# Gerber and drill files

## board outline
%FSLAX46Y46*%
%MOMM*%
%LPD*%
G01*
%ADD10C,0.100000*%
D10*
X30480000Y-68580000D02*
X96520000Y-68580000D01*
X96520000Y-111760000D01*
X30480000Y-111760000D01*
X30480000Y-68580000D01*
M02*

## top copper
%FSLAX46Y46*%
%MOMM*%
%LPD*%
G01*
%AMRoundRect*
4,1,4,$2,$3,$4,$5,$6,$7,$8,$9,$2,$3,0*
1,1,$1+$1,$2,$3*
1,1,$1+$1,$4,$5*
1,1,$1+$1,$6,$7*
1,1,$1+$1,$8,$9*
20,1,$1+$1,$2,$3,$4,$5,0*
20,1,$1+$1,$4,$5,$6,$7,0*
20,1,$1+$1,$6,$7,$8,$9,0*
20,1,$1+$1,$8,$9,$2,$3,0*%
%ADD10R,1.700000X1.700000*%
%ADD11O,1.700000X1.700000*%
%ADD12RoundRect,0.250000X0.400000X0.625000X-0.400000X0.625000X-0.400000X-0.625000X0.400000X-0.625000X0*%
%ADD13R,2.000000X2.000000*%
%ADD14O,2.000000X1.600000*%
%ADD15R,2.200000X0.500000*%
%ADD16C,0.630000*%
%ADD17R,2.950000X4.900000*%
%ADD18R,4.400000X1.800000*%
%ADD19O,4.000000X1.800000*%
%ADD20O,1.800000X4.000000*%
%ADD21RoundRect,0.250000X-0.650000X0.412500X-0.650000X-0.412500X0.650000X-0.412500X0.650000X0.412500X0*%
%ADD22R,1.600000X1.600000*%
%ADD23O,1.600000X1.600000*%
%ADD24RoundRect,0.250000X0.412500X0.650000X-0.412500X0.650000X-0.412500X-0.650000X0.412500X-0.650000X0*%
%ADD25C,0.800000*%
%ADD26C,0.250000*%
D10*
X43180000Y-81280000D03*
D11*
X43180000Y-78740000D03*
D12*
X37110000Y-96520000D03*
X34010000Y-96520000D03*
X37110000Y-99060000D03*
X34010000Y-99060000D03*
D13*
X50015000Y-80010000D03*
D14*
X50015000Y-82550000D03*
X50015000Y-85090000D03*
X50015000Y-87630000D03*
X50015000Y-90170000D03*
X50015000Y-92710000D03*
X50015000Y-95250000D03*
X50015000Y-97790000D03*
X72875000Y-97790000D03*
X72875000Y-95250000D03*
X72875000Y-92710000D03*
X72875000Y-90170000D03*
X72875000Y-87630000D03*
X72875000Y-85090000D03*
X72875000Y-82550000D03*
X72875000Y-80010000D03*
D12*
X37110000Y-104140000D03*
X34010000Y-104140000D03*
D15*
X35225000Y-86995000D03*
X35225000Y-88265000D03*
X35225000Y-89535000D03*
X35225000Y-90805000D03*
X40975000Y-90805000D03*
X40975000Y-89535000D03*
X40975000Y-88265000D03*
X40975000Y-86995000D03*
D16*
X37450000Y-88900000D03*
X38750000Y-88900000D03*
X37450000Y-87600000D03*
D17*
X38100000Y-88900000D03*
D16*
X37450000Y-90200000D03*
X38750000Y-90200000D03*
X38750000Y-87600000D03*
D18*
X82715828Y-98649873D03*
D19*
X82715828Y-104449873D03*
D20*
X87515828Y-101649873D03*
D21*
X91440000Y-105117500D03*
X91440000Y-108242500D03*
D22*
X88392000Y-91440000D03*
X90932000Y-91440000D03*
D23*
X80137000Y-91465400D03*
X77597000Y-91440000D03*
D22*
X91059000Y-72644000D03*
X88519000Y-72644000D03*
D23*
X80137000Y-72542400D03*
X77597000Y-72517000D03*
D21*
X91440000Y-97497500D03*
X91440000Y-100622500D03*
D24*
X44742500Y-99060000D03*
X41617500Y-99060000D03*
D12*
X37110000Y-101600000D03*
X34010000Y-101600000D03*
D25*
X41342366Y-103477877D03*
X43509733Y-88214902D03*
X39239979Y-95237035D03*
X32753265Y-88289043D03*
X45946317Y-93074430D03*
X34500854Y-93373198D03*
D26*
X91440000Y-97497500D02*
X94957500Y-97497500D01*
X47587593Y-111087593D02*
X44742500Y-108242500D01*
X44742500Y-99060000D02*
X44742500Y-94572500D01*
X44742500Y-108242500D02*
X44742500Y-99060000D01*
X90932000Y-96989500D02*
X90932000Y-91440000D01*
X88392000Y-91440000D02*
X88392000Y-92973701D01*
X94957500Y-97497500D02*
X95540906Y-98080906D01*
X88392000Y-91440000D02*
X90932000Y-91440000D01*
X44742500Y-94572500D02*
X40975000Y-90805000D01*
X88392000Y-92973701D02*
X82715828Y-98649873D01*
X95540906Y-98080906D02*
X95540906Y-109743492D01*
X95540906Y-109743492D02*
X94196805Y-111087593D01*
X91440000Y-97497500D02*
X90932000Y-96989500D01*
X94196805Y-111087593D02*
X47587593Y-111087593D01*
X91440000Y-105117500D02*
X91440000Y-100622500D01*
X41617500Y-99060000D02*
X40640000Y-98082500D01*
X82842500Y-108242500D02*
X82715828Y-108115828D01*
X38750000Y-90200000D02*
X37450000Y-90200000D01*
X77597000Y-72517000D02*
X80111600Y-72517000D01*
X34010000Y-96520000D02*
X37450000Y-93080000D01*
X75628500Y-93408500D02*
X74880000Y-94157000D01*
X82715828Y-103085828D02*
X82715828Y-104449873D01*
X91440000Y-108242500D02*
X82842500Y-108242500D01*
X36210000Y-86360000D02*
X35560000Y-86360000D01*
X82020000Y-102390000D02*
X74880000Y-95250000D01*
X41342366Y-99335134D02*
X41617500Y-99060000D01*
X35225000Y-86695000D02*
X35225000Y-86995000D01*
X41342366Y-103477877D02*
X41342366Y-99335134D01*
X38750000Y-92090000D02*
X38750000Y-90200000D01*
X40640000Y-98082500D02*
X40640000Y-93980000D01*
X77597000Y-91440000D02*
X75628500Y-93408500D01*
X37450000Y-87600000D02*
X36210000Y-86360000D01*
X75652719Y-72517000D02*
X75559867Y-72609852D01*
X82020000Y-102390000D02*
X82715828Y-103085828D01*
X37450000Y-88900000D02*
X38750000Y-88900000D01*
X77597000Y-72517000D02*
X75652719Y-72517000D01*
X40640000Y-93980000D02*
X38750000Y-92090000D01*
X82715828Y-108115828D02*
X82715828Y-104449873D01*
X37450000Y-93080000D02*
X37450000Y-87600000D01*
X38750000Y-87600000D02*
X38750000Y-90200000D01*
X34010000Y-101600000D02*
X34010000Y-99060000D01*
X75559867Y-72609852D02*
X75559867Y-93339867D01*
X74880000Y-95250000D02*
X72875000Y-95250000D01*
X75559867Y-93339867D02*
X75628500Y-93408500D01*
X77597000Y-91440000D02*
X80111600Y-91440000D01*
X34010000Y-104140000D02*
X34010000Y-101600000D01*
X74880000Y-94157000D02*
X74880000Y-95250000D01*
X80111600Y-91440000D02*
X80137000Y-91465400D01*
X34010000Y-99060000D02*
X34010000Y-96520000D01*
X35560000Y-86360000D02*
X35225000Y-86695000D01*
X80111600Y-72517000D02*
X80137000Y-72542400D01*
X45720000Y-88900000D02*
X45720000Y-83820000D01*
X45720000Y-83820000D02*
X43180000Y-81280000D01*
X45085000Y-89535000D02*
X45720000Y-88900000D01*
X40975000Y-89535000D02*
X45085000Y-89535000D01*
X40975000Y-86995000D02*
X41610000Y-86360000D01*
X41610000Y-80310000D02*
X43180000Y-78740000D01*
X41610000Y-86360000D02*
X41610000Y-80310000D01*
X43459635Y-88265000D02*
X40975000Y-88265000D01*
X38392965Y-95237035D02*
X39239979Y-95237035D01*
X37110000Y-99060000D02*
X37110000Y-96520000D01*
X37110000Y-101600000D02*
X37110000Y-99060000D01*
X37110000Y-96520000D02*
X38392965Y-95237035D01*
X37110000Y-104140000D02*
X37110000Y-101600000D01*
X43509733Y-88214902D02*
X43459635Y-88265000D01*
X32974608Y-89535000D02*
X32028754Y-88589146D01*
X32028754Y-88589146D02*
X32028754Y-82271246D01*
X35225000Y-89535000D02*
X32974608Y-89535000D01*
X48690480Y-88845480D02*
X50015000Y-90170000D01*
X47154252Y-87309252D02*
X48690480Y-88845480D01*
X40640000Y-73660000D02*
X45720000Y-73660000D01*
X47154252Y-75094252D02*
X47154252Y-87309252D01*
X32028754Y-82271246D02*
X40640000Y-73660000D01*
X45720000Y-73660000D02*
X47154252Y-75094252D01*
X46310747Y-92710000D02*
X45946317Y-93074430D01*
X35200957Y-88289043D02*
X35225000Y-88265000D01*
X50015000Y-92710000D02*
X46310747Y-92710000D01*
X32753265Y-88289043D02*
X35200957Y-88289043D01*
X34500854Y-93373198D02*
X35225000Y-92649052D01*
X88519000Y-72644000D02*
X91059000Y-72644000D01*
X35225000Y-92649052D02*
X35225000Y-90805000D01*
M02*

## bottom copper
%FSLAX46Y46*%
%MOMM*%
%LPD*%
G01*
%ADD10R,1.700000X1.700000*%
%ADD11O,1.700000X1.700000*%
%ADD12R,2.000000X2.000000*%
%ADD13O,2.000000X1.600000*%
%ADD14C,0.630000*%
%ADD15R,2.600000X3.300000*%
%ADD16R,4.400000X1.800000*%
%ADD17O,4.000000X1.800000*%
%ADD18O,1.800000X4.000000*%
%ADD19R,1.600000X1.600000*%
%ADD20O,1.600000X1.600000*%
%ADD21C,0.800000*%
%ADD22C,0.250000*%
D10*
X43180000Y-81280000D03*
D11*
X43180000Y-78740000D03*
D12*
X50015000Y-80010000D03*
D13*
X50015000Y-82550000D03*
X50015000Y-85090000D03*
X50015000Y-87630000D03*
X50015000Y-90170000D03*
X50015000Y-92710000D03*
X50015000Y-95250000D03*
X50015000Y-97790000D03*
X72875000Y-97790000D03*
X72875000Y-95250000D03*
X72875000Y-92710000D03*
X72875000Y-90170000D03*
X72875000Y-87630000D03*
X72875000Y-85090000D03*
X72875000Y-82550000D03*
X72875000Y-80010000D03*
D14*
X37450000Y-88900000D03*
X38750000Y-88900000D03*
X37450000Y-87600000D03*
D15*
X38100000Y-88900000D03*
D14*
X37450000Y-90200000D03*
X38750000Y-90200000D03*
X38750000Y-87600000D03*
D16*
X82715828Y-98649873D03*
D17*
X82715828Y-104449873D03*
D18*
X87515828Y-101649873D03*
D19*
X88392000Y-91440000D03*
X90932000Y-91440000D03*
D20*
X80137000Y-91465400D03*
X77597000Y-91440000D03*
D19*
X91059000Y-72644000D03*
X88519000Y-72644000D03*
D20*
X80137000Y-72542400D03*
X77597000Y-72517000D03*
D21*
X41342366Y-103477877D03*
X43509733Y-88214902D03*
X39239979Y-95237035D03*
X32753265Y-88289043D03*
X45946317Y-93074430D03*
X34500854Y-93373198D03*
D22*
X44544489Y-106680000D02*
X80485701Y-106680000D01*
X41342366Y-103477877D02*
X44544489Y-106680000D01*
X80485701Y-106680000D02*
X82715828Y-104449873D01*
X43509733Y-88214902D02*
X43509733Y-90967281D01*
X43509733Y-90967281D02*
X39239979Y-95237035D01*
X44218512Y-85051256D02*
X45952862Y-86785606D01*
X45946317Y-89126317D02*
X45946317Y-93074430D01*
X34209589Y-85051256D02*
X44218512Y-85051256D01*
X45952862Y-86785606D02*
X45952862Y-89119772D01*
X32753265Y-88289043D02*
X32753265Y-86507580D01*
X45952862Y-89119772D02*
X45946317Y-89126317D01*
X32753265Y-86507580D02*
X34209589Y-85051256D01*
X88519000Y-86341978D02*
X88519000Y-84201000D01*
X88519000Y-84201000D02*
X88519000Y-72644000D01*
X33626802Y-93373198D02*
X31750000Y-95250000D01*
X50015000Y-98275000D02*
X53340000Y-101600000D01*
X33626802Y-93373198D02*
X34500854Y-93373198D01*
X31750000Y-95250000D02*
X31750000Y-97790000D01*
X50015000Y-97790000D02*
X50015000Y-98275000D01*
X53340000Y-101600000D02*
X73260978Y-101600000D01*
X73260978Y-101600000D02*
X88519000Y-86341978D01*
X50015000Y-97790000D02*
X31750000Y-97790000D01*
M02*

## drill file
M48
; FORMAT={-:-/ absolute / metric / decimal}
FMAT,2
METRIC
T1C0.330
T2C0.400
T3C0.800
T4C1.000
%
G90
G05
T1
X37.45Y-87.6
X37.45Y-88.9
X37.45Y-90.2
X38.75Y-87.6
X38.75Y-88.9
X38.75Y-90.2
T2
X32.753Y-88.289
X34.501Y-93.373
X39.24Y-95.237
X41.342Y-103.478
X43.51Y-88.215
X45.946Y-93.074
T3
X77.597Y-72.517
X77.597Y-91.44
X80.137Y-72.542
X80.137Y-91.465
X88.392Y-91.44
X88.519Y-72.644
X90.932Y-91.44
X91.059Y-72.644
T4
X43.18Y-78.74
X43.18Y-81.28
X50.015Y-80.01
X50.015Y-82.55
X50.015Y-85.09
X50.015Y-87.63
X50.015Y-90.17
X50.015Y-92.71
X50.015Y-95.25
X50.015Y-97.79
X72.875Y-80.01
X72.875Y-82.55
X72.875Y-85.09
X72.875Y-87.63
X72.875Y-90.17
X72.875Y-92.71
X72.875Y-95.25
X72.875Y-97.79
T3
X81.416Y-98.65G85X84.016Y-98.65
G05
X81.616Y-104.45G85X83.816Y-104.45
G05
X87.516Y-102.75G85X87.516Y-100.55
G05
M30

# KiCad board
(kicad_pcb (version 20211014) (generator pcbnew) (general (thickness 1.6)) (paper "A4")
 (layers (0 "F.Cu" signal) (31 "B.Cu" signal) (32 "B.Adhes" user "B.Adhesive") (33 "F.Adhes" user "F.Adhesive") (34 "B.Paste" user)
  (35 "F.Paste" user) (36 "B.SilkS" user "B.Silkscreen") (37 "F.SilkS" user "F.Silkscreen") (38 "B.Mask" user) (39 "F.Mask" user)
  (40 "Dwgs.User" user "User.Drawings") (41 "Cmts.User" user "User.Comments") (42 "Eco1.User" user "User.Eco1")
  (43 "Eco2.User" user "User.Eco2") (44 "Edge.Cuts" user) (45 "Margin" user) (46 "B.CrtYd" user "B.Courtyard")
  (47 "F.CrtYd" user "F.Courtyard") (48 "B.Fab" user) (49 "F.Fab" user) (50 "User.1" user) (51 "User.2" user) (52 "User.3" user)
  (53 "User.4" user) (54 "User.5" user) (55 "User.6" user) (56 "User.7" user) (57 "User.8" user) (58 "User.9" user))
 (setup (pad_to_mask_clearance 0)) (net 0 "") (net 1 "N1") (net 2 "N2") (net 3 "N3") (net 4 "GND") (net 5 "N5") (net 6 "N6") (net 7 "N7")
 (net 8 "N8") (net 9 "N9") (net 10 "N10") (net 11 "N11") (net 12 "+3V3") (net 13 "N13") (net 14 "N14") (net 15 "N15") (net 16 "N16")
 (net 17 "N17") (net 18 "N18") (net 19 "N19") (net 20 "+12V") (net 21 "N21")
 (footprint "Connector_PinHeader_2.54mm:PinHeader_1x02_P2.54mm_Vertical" (layer "F.Cu") (at 43.18 81.28 180)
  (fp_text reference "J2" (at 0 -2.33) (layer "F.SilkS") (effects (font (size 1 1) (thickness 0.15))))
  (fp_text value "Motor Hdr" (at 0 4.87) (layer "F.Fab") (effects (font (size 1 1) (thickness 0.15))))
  (pad "1" thru_hole rect (at 0 0 180) (size 1.7 1.7) (drill 1) (layers *.Cu *.Mask) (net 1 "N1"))
  (pad "2" thru_hole oval (at 0 2.54 180) (size 1.7 1.7) (drill 1) (layers *.Cu *.Mask) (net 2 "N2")))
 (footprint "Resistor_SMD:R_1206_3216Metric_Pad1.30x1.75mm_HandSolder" (layer "F.Cu") (at 35.56 96.52 180)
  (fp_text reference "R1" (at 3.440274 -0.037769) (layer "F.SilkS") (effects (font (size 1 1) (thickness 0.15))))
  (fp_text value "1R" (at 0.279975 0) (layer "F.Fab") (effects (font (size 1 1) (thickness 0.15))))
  (pad "1" smd roundrect (at -1.55 0 180) (size 1.3 1.75) (layers "F.Cu" "F.Paste" "F.Mask") (roundrect_rratio 0.1923076923) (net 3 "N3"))
  (pad "2" smd roundrect (at 1.55 0 180) (size 1.3 1.75) (layers "F.Cu" "F.Paste" "F.Mask") (roundrect_rratio 0.1923076923) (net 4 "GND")))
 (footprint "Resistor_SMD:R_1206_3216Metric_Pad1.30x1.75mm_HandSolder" (layer "F.Cu") (at 35.56 99.06 180)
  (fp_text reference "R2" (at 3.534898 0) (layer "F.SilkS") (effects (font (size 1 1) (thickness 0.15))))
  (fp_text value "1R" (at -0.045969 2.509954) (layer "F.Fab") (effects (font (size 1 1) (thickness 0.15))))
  (pad "1" smd roundrect (at -1.55 0 180) (size 1.3 1.75) (layers "F.Cu" "F.Paste" "F.Mask") (roundrect_rratio 0.1923076923) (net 3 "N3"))
  (pad "2" smd roundrect (at 1.55 0 180) (size 1.3 1.75) (layers "F.Cu" "F.Paste" "F.Mask") (roundrect_rratio 0.1923076923) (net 4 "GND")))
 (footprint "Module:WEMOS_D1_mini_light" (layer "F.Cu") (at 50.015 80.01)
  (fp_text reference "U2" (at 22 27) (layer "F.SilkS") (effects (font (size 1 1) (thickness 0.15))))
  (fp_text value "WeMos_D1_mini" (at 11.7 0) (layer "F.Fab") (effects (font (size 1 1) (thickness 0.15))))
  (pad "1" thru_hole rect (at 0 0) (size 2 2) (drill 1) (layers *.Cu *.Mask) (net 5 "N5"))
  (pad "2" thru_hole oval (at 0 2.54) (size 2 1.6) (drill 1) (layers *.Cu *.Mask) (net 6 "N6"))
  (pad "3" thru_hole oval (at 0 5.08) (size 2 1.6) (drill 1) (layers *.Cu *.Mask) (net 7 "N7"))
  (pad "4" thru_hole oval (at 0 7.62) (size 2 1.6) (drill 1) (layers *.Cu *.Mask) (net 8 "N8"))
  (pad "5" thru_hole oval (at 0 10.16) (size 2 1.6) (drill 1) (layers *.Cu *.Mask) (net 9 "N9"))
  (pad "6" thru_hole oval (at 0 12.7) (size 2 1.6) (drill 1) (layers *.Cu *.Mask) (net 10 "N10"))
  (pad "7" thru_hole oval (at 0 15.24) (size 2 1.6) (drill 1) (layers *.Cu *.Mask) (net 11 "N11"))
  (pad "8" thru_hole oval (at 0 17.78) (size 2 1.6) (drill 1) (layers *.Cu *.Mask) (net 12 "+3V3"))
  (pad "9" thru_hole oval (at 22.86 17.78) (size 2 1.6) (drill 1) (layers *.Cu *.Mask) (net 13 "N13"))
  (pad "10" thru_hole oval (at 22.86 15.24) (size 2 1.6) (drill 1) (layers *.Cu *.Mask) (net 4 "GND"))
  (pad "11" thru_hole oval (at 22.86 12.7) (size 2 1.6) (drill 1) (layers *.Cu *.Mask) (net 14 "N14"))
  (pad "12" thru_hole oval (at 22.86 10.16) (size 2 1.6) (drill 1) (layers *.Cu *.Mask) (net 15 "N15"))
  (pad "13" thru_hole oval (at 22.86 7.62) (size 2 1.6) (drill 1) (layers *.Cu *.Mask) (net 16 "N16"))
  (pad "14" thru_hole oval (at 22.86 5.08) (size 2 1.6) (drill 1) (layers *.Cu *.Mask) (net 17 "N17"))
  (pad "15" thru_hole oval (at 22.86 2.54) (size 2 1.6) (drill 1) (layers *.Cu *.Mask) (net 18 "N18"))
  (pad "16" thru_hole oval (at 22.86 0) (size 2 1.6) (drill 1) (layers *.Cu *.Mask) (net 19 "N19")))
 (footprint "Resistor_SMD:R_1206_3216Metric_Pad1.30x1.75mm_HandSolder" (layer "F.Cu") (at 35.56 104.14 180)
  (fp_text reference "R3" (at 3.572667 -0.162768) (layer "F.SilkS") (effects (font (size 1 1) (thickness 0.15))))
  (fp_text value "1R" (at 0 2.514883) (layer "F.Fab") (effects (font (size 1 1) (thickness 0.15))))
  (pad "1" smd roundrect (at -1.55 0 180) (size 1.3 1.75) (layers "F.Cu" "F.Paste" "F.Mask") (roundrect_rratio 0.1923076923) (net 3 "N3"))
  (pad "2" smd roundrect (at 1.55 0 180) (size 1.3 1.75) (layers "F.Cu" "F.Paste" "F.Mask") (roundrect_rratio 0.1923076923) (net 4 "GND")))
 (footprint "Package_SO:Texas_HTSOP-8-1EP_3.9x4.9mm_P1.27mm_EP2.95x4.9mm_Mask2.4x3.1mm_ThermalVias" (layer "F.Cu") (at 38.1 88.9)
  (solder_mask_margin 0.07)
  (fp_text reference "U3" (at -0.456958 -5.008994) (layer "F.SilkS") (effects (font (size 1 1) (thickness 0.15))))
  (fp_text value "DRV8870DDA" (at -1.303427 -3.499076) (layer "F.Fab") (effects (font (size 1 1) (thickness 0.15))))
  (pad "" smd rect (at 0 0) (size 2.4 3.1) (layers "F.Mask")) (pad "" smd rect (at 0 0) (size 2.4 3.1) (layers "F.Paste"))
  (pad "1" smd rect (at -2.875 -1.905) (size 2.2 0.5) (layers "F.Cu" "F.Paste" "F.Mask") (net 4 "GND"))
  (pad "2" smd rect (at -2.875 -0.635) (size 2.2 0.5) (layers "F.Cu" "F.Paste" "F.Mask") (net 10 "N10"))
  (pad "3" smd rect (at -2.875 0.635) (size 2.2 0.5) (layers "F.Cu" "F.Paste" "F.Mask") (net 9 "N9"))
  (pad "4" smd rect (at -2.875 1.905) (size 2.2 0.5) (layers "F.Cu" "F.Paste" "F.Mask") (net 12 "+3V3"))
  (pad "5" smd rect (at 2.875 1.905) (size 2.2 0.5) (layers "F.Cu" "F.Paste" "F.Mask") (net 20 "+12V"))
  (pad "6" smd rect (at 2.875 0.635) (size 2.2 0.5) (layers "F.Cu" "F.Paste" "F.Mask") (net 1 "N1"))
  (pad "7" smd rect (at 2.875 -0.635) (size 2.2 0.5) (layers "F.Cu" "F.Paste" "F.Mask") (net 3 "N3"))
  (pad "8" smd rect (at 2.875 -1.905) (size 2.2 0.5) (layers "F.Cu" "F.Paste" "F.Mask") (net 2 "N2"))
  (pad "9" thru_hole circle (at -0.65 0) (size 0.63 0.63) (drill 0.33) (layers *.Cu *.Mask) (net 4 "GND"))
  (pad "9" thru_hole circle (at 0.65 0) (size 0.63 0.63) (drill 0.33) (layers *.Cu *.Mask) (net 4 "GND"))
  (pad "9" thru_hole circle (at -0.65 -1.3) (size 0.63 0.63) (drill 0.33) (layers *.Cu *.Mask) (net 4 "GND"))
  (pad "9" smd rect (at 0 0) (size 2.6 3.3) (layers "B.Cu") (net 4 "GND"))
  (pad "9" smd rect (at 0 0) (size 2.95 4.9) (layers "F.Cu") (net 4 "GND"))
  (pad "9" thru_hole circle (at -0.65 1.3) (size 0.63 0.63) (drill 0.33) (layers *.Cu *.Mask) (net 4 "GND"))
  (pad "9" thru_hole circle (at 0.65 1.3) (size 0.63 0.63) (drill 0.33) (layers *.Cu *.Mask) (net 4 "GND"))
  (pad "9" thru_hole circle (at 0.65 -1.3) (size 0.63 0.63) (drill 0.33) (layers *.Cu *.Mask) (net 4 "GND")))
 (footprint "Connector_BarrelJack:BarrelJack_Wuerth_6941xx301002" (layer "F.Cu") (at 82.715828 98.649873)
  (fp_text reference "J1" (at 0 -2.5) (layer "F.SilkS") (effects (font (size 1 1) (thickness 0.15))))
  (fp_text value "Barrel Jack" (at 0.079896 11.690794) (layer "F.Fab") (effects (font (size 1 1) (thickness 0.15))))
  (pad "1" thru_hole rect (at 0 0) (size 4.4 1.8) (drill oval 3.4 0.8) (layers *.Cu *.Mask) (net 20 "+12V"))
  (pad "2" thru_hole oval (at 0 5.8) (size 4 1.8) (drill oval 3 0.8) (layers *.Cu *.Mask) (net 4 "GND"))
  (pad "3" thru_hole oval (at 4.8 3 90) (size 4 1.8) (drill oval 3 0.8) (layers *.Cu *.Mask)))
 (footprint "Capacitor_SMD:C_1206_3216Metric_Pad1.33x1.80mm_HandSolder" (layer "F.Cu") (at 91.44 106.68 -90)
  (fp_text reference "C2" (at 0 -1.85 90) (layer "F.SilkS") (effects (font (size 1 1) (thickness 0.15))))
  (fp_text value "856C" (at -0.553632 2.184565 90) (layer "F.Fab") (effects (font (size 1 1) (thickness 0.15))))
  (pad "1" smd roundrect (at -1.5625 0 270) (size 1.325 1.8) (layers "F.Cu" "F.Paste" "F.Mask") (roundrect_rratio 0.1886792453)
   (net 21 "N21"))
  (pad "2" smd roundrect (at 1.5625 0 270) (size 1.325 1.8) (layers "F.Cu" "F.Paste" "F.Mask") (roundrect_rratio 0.1886792453) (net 4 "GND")))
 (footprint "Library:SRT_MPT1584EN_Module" (layer "F.Cu") (at 83.82 81.28 90)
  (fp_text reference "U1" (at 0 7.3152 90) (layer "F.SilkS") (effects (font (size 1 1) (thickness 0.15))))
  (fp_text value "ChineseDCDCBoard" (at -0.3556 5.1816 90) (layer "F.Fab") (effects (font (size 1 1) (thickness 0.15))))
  (pad "1" thru_hole rect (at -10.16 4.572 180) (size 1.6 1.6) (drill 0.8) (layers *.Cu "B.Mask") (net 20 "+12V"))
  (pad "1" thru_hole rect (at -10.16 7.112 180) (size 1.6 1.6) (drill 0.8) (layers *.Cu "B.Mask") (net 20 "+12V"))
  (pad "2" thru_hole oval (at -10.1854 -3.683 180) (size 1.6 1.6) (drill 0.8) (layers *.Cu "B.Mask") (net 4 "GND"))
  (pad "2" thru_hole oval (at -10.16 -6.223 180) (size 1.6 1.6) (drill 0.8) (layers *.Cu "B.Mask") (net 4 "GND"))
  (pad "3" thru_hole rect (at 8.636 7.239 180) (size 1.6 1.6) (drill 0.8) (layers *.Cu "B.Mask") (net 12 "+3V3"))
  (pad "3" thru_hole rect (at 8.636 4.699 180) (size 1.6 1.6) (drill 0.8) (layers *.Cu "B.Mask") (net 12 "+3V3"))
  (pad "4" thru_hole oval (at 8.7376 -3.683 180) (size 1.6 1.6) (drill 0.8) (layers *.Cu "B.Mask") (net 4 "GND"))
  (pad "4" thru_hole oval (at 8.763 -6.223 180) (size 1.6 1.6) (drill 0.8) (layers *.Cu "B.Mask") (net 4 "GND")))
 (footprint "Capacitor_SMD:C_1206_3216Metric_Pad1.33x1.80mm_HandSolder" (layer "F.Cu") (at 91.44 99.06 -90)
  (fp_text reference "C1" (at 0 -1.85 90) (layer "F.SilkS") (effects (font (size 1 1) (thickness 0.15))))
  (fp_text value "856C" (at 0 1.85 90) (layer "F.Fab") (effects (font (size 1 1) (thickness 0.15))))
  (pad "1" smd roundrect (at -1.5625 0 270) (size 1.325 1.8) (layers "F.Cu" "F.Paste" "F.Mask") (roundrect_rratio 0.1886792453)
   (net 20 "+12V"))
  (pad "2" smd roundrect (at 1.5625 0 270) (size 1.325 1.8) (layers "F.Cu" "F.Paste" "F.Mask") (roundrect_rratio 0.1886792453)
   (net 21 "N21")))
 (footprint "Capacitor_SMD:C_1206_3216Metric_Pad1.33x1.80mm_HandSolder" (layer "F.Cu") (at 43.18 99.06 180)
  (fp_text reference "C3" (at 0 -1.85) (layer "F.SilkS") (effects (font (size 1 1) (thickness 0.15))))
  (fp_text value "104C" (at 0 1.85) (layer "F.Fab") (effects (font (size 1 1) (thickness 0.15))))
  (pad "1" smd roundrect (at -1.5625 0 180) (size 1.325 1.8) (layers "F.Cu" "F.Paste" "F.Mask") (roundrect_rratio 0.1886792453)
   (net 20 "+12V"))
  (pad "2" smd roundrect (at 1.5625 0 180) (size 1.325 1.8) (layers "F.Cu" "F.Paste" "F.Mask") (roundrect_rratio 0.1886792453) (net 4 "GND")))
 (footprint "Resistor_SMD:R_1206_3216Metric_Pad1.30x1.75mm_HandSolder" (layer "F.Cu") (at 35.56 101.6 180)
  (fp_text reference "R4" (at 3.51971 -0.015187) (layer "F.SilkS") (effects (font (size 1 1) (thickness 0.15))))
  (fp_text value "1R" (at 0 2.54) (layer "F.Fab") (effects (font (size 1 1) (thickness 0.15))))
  (pad "1" smd roundrect (at -1.55 0 180) (size 1.3 1.75) (layers "F.Cu" "F.Paste" "F.Mask") (roundrect_rratio 0.1923076923) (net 3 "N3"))
  (pad "2" smd roundrect (at 1.55 0 180) (size 1.3 1.75) (layers "F.Cu" "F.Paste" "F.Mask") (roundrect_rratio 0.1923076923) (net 4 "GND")))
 (gr_rect (start 96.52 111.76) (end 30.48 68.58) (layer "Edge.Cuts") (width 0.1) (fill none))
 (segment (start 91.44 97.4975) (end 94.9575 97.4975) (width 0.25) (layer "F.Cu") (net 20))
 (segment (start 47.587593 111.087593) (end 44.7425 108.2425) (width 0.25) (layer "F.Cu") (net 20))
 (segment (start 44.7425 99.06) (end 44.7425 94.5725) (width 0.25) (layer "F.Cu") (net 20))
 (segment (start 44.7425 108.2425) (end 44.7425 99.06) (width 0.25) (layer "F.Cu") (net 20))
 (segment (start 90.932 96.9895) (end 90.932 91.44) (width 0.25) (layer "F.Cu") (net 20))
 (segment (start 88.392 91.44) (end 88.392 92.973701) (width 0.25) (layer "F.Cu") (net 20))
 (segment (start 94.9575 97.4975) (end 95.540906 98.080906) (width 0.25) (layer "F.Cu") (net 20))
 (segment (start 88.392 91.44) (end 90.932 91.44) (width 0.25) (layer "F.Cu") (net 20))
 (segment (start 44.7425 94.5725) (end 40.975 90.805) (width 0.25) (layer "F.Cu") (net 20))
 (segment (start 88.392 92.973701) (end 82.715828 98.649873) (width 0.25) (layer "F.Cu") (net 20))
 (segment (start 95.540906 98.080906) (end 95.540906 109.743492) (width 0.25) (layer "F.Cu") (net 20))
 (segment (start 95.540906 109.743492) (end 94.196805 111.087593) (width 0.25) (layer "F.Cu") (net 20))
 (segment (start 91.44 97.4975) (end 90.932 96.9895) (width 0.25) (layer "F.Cu") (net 20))
 (segment (start 94.196805 111.087593) (end 47.587593 111.087593) (width 0.25) (layer "F.Cu") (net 20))
 (segment (start 91.44 105.1175) (end 91.44 100.6225) (width 0.25) (layer "F.Cu") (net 21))
 (segment (start 41.6175 99.06) (end 40.64 98.0825) (width 0.25) (layer "F.Cu") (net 4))
 (segment (start 82.8425 108.2425) (end 82.715828 108.115828) (width 0.25) (layer "F.Cu") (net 4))
 (segment (start 38.75 90.2) (end 37.45 90.2) (width 0.25) (layer "F.Cu") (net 4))
 (segment (start 77.597 72.517) (end 80.1116 72.517) (width 0.25) (layer "F.Cu") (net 4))
 (segment (start 34.01 96.52) (end 37.45 93.08) (width 0.25) (layer "F.Cu") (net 4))
 (segment (start 75.6285 93.4085) (end 74.88 94.157) (width 0.25) (layer "F.Cu") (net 4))
 (segment (start 82.715828 103.085828) (end 82.715828 104.449873) (width 0.25) (layer "F.Cu") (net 4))
 (segment (start 91.44 108.2425) (end 82.8425 108.2425) (width 0.25) (layer "F.Cu") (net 4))
 (segment (start 36.21 86.36) (end 35.56 86.36) (width 0.25) (layer "F.Cu") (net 4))
 (segment (start 82.02 102.39) (end 74.88 95.25) (width 0.25) (layer "F.Cu") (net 4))
 (segment (start 41.342366 99.335134) (end 41.6175 99.06) (width 0.25) (layer "F.Cu") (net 4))
 (segment (start 35.225 86.695) (end 35.225 86.995) (width 0.25) (layer "F.Cu") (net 4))
 (segment (start 41.342366 103.477877) (end 41.342366 99.335134) (width 0.25) (layer "F.Cu") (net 4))
 (segment (start 38.75 92.09) (end 38.75 90.2) (width 0.25) (layer "F.Cu") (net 4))
 (segment (start 40.64 98.0825) (end 40.64 93.98) (width 0.25) (layer "F.Cu") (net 4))
 (segment (start 77.597 91.44) (end 75.6285 93.4085) (width 0.25) (layer "F.Cu") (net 4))
 (segment (start 37.45 87.6) (end 36.21 86.36) (width 0.25) (layer "F.Cu") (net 4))
 (segment (start 75.652719 72.517) (end 75.559867 72.609852) (width 0.25) (layer "F.Cu") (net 4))
 (segment (start 82.02 102.39) (end 82.715828 103.085828) (width 0.25) (layer "F.Cu") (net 4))
 (segment (start 37.45 88.9) (end 38.75 88.9) (width 0.25) (layer "F.Cu") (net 4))
 (segment (start 77.597 72.517) (end 75.652719 72.517) (width 0.25) (layer "F.Cu") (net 4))
 (segment (start 40.64 93.98) (end 38.75 92.09) (width 0.25) (layer "F.Cu") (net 4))
 (segment (start 82.715828 108.115828) (end 82.715828 104.449873) (width 0.25) (layer "F.Cu") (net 4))
 (segment (start 37.45 93.08) (end 37.45 87.6) (width 0.25) (layer "F.Cu") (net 4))
 (segment (start 38.75 87.6) (end 38.75 90.2) (width 0.25) (layer "F.Cu") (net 4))
 (segment (start 34.01 101.6) (end 34.01 99.06) (width 0.25) (layer "F.Cu") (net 4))
 (segment (start 75.559867 72.609852) (end 75.559867 93.339867) (width 0.25) (layer "F.Cu") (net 4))
 (segment (start 74.88 95.25) (end 72.875 95.25) (width 0.25) (layer "F.Cu") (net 4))
 (segment (start 75.559867 93.339867) (end 75.6285 93.4085) (width 0.25) (layer "F.Cu") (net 4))
 (segment (start 77.597 91.44) (end 80.1116 91.44) (width 0.25) (layer "F.Cu") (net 4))
 (segment (start 34.01 104.14) (end 34.01 101.6) (width 0.25) (layer "F.Cu") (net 4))
 (segment (start 74.88 94.157) (end 74.88 95.25) (width 0.25) (layer "F.Cu") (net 4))
 (segment (start 80.1116 91.44) (end 80.137 91.4654) (width 0.25) (layer "F.Cu") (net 4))
 (segment (start 34.01 99.06) (end 34.01 96.52) (width 0.25) (layer "F.Cu") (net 4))
 (segment (start 35.56 86.36) (end 35.225 86.695) (width 0.25) (layer "F.Cu") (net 4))
 (segment (start 80.1116 72.517) (end 80.137 72.5424) (width 0.25) (layer "F.Cu") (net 4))
 (via (at 41.342366 103.477877) (size 0.8) (drill 0.4) (layers "F.Cu" "B.Cu") (free) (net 4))
 (segment (start 44.544489 106.68) (end 80.485701 106.68) (width 0.25) (layer "B.Cu") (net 4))
 (segment (start 41.342366 103.477877) (end 44.544489 106.68) (width 0.25) (layer "B.Cu") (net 4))
 (segment (start 80.485701 106.68) (end 82.715828 104.449873) (width 0.25) (layer "B.Cu") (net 4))
 (segment (start 45.72 88.9) (end 45.72 83.82) (width 0.25) (layer "F.Cu") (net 1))
 (segment (start 45.72 83.82) (end 43.18 81.28) (width 0.25) (layer "F.Cu") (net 1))
 (segment (start 45.085 89.535) (end 45.72 88.9) (width 0.25) (layer "F.Cu") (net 1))
 (segment (start 40.975 89.535) (end 45.085 89.535) (width 0.25) (layer "F.Cu") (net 1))
 (segment (start 40.975 86.995) (end 41.61 86.36) (width 0.25) (layer "F.Cu") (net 2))
 (segment (start 41.61 80.31) (end 43.18 78.74) (width 0.25) (layer "F.Cu") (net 2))
 (segment (start 41.61 86.36) (end 41.61 80.31) (width 0.25) (layer "F.Cu") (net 2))
 (segment (start 43.459635 88.265) (end 40.975 88.265) (width 0.25) (layer "F.Cu") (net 3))
 (segment (start 38.392965 95.237035) (end 39.239979 95.237035) (width 0.25) (layer "F.Cu") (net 3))
 (segment (start 37.11 99.06) (end 37.11 96.52) (width 0.25) (layer "F.Cu") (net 3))
 (segment (start 37.11 101.6) (end 37.11 99.06) (width 0.25) (layer "F.Cu") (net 3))
 (segment (start 37.11 96.52) (end 38.392965 95.237035) (width 0.25) (layer "F.Cu") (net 3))
 (segment (start 37.11 104.14) (end 37.11 101.6) (width 0.25) (layer "F.Cu") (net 3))
 (segment (start 43.509733 88.214902) (end 43.459635 88.265) (width 0.25) (layer "F.Cu") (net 3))
 (via (at 43.509733 88.214902) (size 0.8) (drill 0.4) (layers "F.Cu" "B.Cu") (free) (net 3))
 (via (at 39.239979 95.237035) (size 0.8) (drill 0.4) (layers "F.Cu" "B.Cu") (free) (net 3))
 (segment (start 43.509733 88.214902) (end 43.509733 90.967281) (width 0.25) (layer "B.Cu") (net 3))
 (segment (start 43.509733 90.967281) (end 39.239979 95.237035) (width 0.25) (layer "B.Cu") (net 3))
 (segment (start 32.974608 89.535) (end 32.028754 88.589146) (width 0.25) (layer "F.Cu") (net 9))
 (segment (start 32.028754 88.589146) (end 32.028754 82.271246) (width 0.25) (layer "F.Cu") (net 9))
 (segment (start 35.225 89.535) (end 32.974608 89.535) (width 0.25) (layer "F.Cu") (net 9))
 (segment (start 48.69048 88.84548) (end 50.015 90.17) (width 0.25) (layer "F.Cu") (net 9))
 (segment (start 47.154252 87.309252) (end 48.69048 88.84548) (width 0.25) (layer "F.Cu") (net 9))
 (segment (start 40.64 73.66) (end 45.72 73.66) (width 0.25) (layer "F.Cu") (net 9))
 (segment (start 47.154252 75.094252) (end 47.154252 87.309252) (width 0.25) (layer "F.Cu") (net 9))
 (segment (start 32.028754 82.271246) (end 40.64 73.66) (width 0.25) (layer "F.Cu") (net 9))
 (segment (start 45.72 73.66) (end 47.154252 75.094252) (width 0.25) (layer "F.Cu") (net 9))
 (segment (start 46.310747 92.71) (end 45.946317 93.07443) (width 0.25) (layer "F.Cu") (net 10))
 (segment (start 35.200957 88.289043) (end 35.225 88.265) (width 0.25) (layer "F.Cu") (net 10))
 (segment (start 50.015 92.71) (end 46.310747 92.71) (width 0.25) (layer "F.Cu") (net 10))
 (segment (start 32.753265 88.289043) (end 35.200957 88.289043) (width 0.25) (layer "F.Cu") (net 10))
 (via (at 32.753265 88.289043) (size 0.8) (drill 0.4) (layers "F.Cu" "B.Cu") (free) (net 10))
 (via (at 45.946317 93.07443) (size 0.8) (drill 0.4) (layers "F.Cu" "B.Cu") (free) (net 10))
 (segment (start 44.218512 85.051256) (end 45.952862 86.785606) (width 0.25) (layer "B.Cu") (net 10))
 (segment (start 45.946317 89.126317) (end 45.946317 93.07443) (width 0.25) (layer "B.Cu") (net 10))
 (segment (start 34.209589 85.051256) (end 44.218512 85.051256) (width 0.25) (layer "B.Cu") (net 10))
 (segment (start 45.952862 86.785606) (end 45.952862 89.119772) (width 0.25) (layer "B.Cu") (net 10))
 (segment (start 32.753265 88.289043) (end 32.753265 86.50758) (width 0.25) (layer "B.Cu") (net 10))
 (segment (start 45.952862 89.119772) (end 45.946317 89.126317) (width 0.25) (layer "B.Cu") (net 10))
 (segment (start 32.753265 86.50758) (end 34.209589 85.051256) (width 0.25) (layer "B.Cu") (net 10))
 (segment (start 34.500854 93.373198) (end 35.225 92.649052) (width 0.25) (layer "F.Cu") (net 12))
 (segment (start 88.519 72.644) (end 91.059 72.644) (width 0.25) (layer "F.Cu") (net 12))
 (segment (start 35.225 92.649052) (end 35.225 90.805) (width 0.25) (layer "F.Cu") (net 12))
 (via (at 34.500854 93.373198) (size 0.8) (drill 0.4) (layers "F.Cu" "B.Cu") (free) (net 12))
 (segment (start 88.519 86.341978) (end 88.519 84.201) (width 0.25) (layer "B.Cu") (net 12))
 (segment (start 88.519 84.201) (end 88.519 72.644) (width 0.25) (layer "B.Cu") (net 12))
 (segment (start 33.626802 93.373198) (end 31.75 95.25) (width 0.25) (layer "B.Cu") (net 12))
 (segment (start 50.015 98.275) (end 53.34 101.6) (width 0.25) (layer "B.Cu") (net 12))
 (segment (start 33.626802 93.373198) (end 34.500854 93.373198) (width 0.25) (layer "B.Cu") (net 12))
 (segment (start 31.75 95.25) (end 31.75 97.79) (width 0.25) (layer "B.Cu") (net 12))
 (segment (start 50.015 97.79) (end 50.015 98.275) (width 0.25) (layer "B.Cu") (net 12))
 (segment (start 53.34 101.6) (end 73.260978 101.6) (width 0.25) (layer "B.Cu") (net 12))
 (segment (start 73.260978 101.6) (end 88.519 86.341978) (width 0.25) (layer "B.Cu") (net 12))
 (segment (start 50.015 97.79) (end 31.75 97.79) (width 0.25) (layer "B.Cu") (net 12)))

